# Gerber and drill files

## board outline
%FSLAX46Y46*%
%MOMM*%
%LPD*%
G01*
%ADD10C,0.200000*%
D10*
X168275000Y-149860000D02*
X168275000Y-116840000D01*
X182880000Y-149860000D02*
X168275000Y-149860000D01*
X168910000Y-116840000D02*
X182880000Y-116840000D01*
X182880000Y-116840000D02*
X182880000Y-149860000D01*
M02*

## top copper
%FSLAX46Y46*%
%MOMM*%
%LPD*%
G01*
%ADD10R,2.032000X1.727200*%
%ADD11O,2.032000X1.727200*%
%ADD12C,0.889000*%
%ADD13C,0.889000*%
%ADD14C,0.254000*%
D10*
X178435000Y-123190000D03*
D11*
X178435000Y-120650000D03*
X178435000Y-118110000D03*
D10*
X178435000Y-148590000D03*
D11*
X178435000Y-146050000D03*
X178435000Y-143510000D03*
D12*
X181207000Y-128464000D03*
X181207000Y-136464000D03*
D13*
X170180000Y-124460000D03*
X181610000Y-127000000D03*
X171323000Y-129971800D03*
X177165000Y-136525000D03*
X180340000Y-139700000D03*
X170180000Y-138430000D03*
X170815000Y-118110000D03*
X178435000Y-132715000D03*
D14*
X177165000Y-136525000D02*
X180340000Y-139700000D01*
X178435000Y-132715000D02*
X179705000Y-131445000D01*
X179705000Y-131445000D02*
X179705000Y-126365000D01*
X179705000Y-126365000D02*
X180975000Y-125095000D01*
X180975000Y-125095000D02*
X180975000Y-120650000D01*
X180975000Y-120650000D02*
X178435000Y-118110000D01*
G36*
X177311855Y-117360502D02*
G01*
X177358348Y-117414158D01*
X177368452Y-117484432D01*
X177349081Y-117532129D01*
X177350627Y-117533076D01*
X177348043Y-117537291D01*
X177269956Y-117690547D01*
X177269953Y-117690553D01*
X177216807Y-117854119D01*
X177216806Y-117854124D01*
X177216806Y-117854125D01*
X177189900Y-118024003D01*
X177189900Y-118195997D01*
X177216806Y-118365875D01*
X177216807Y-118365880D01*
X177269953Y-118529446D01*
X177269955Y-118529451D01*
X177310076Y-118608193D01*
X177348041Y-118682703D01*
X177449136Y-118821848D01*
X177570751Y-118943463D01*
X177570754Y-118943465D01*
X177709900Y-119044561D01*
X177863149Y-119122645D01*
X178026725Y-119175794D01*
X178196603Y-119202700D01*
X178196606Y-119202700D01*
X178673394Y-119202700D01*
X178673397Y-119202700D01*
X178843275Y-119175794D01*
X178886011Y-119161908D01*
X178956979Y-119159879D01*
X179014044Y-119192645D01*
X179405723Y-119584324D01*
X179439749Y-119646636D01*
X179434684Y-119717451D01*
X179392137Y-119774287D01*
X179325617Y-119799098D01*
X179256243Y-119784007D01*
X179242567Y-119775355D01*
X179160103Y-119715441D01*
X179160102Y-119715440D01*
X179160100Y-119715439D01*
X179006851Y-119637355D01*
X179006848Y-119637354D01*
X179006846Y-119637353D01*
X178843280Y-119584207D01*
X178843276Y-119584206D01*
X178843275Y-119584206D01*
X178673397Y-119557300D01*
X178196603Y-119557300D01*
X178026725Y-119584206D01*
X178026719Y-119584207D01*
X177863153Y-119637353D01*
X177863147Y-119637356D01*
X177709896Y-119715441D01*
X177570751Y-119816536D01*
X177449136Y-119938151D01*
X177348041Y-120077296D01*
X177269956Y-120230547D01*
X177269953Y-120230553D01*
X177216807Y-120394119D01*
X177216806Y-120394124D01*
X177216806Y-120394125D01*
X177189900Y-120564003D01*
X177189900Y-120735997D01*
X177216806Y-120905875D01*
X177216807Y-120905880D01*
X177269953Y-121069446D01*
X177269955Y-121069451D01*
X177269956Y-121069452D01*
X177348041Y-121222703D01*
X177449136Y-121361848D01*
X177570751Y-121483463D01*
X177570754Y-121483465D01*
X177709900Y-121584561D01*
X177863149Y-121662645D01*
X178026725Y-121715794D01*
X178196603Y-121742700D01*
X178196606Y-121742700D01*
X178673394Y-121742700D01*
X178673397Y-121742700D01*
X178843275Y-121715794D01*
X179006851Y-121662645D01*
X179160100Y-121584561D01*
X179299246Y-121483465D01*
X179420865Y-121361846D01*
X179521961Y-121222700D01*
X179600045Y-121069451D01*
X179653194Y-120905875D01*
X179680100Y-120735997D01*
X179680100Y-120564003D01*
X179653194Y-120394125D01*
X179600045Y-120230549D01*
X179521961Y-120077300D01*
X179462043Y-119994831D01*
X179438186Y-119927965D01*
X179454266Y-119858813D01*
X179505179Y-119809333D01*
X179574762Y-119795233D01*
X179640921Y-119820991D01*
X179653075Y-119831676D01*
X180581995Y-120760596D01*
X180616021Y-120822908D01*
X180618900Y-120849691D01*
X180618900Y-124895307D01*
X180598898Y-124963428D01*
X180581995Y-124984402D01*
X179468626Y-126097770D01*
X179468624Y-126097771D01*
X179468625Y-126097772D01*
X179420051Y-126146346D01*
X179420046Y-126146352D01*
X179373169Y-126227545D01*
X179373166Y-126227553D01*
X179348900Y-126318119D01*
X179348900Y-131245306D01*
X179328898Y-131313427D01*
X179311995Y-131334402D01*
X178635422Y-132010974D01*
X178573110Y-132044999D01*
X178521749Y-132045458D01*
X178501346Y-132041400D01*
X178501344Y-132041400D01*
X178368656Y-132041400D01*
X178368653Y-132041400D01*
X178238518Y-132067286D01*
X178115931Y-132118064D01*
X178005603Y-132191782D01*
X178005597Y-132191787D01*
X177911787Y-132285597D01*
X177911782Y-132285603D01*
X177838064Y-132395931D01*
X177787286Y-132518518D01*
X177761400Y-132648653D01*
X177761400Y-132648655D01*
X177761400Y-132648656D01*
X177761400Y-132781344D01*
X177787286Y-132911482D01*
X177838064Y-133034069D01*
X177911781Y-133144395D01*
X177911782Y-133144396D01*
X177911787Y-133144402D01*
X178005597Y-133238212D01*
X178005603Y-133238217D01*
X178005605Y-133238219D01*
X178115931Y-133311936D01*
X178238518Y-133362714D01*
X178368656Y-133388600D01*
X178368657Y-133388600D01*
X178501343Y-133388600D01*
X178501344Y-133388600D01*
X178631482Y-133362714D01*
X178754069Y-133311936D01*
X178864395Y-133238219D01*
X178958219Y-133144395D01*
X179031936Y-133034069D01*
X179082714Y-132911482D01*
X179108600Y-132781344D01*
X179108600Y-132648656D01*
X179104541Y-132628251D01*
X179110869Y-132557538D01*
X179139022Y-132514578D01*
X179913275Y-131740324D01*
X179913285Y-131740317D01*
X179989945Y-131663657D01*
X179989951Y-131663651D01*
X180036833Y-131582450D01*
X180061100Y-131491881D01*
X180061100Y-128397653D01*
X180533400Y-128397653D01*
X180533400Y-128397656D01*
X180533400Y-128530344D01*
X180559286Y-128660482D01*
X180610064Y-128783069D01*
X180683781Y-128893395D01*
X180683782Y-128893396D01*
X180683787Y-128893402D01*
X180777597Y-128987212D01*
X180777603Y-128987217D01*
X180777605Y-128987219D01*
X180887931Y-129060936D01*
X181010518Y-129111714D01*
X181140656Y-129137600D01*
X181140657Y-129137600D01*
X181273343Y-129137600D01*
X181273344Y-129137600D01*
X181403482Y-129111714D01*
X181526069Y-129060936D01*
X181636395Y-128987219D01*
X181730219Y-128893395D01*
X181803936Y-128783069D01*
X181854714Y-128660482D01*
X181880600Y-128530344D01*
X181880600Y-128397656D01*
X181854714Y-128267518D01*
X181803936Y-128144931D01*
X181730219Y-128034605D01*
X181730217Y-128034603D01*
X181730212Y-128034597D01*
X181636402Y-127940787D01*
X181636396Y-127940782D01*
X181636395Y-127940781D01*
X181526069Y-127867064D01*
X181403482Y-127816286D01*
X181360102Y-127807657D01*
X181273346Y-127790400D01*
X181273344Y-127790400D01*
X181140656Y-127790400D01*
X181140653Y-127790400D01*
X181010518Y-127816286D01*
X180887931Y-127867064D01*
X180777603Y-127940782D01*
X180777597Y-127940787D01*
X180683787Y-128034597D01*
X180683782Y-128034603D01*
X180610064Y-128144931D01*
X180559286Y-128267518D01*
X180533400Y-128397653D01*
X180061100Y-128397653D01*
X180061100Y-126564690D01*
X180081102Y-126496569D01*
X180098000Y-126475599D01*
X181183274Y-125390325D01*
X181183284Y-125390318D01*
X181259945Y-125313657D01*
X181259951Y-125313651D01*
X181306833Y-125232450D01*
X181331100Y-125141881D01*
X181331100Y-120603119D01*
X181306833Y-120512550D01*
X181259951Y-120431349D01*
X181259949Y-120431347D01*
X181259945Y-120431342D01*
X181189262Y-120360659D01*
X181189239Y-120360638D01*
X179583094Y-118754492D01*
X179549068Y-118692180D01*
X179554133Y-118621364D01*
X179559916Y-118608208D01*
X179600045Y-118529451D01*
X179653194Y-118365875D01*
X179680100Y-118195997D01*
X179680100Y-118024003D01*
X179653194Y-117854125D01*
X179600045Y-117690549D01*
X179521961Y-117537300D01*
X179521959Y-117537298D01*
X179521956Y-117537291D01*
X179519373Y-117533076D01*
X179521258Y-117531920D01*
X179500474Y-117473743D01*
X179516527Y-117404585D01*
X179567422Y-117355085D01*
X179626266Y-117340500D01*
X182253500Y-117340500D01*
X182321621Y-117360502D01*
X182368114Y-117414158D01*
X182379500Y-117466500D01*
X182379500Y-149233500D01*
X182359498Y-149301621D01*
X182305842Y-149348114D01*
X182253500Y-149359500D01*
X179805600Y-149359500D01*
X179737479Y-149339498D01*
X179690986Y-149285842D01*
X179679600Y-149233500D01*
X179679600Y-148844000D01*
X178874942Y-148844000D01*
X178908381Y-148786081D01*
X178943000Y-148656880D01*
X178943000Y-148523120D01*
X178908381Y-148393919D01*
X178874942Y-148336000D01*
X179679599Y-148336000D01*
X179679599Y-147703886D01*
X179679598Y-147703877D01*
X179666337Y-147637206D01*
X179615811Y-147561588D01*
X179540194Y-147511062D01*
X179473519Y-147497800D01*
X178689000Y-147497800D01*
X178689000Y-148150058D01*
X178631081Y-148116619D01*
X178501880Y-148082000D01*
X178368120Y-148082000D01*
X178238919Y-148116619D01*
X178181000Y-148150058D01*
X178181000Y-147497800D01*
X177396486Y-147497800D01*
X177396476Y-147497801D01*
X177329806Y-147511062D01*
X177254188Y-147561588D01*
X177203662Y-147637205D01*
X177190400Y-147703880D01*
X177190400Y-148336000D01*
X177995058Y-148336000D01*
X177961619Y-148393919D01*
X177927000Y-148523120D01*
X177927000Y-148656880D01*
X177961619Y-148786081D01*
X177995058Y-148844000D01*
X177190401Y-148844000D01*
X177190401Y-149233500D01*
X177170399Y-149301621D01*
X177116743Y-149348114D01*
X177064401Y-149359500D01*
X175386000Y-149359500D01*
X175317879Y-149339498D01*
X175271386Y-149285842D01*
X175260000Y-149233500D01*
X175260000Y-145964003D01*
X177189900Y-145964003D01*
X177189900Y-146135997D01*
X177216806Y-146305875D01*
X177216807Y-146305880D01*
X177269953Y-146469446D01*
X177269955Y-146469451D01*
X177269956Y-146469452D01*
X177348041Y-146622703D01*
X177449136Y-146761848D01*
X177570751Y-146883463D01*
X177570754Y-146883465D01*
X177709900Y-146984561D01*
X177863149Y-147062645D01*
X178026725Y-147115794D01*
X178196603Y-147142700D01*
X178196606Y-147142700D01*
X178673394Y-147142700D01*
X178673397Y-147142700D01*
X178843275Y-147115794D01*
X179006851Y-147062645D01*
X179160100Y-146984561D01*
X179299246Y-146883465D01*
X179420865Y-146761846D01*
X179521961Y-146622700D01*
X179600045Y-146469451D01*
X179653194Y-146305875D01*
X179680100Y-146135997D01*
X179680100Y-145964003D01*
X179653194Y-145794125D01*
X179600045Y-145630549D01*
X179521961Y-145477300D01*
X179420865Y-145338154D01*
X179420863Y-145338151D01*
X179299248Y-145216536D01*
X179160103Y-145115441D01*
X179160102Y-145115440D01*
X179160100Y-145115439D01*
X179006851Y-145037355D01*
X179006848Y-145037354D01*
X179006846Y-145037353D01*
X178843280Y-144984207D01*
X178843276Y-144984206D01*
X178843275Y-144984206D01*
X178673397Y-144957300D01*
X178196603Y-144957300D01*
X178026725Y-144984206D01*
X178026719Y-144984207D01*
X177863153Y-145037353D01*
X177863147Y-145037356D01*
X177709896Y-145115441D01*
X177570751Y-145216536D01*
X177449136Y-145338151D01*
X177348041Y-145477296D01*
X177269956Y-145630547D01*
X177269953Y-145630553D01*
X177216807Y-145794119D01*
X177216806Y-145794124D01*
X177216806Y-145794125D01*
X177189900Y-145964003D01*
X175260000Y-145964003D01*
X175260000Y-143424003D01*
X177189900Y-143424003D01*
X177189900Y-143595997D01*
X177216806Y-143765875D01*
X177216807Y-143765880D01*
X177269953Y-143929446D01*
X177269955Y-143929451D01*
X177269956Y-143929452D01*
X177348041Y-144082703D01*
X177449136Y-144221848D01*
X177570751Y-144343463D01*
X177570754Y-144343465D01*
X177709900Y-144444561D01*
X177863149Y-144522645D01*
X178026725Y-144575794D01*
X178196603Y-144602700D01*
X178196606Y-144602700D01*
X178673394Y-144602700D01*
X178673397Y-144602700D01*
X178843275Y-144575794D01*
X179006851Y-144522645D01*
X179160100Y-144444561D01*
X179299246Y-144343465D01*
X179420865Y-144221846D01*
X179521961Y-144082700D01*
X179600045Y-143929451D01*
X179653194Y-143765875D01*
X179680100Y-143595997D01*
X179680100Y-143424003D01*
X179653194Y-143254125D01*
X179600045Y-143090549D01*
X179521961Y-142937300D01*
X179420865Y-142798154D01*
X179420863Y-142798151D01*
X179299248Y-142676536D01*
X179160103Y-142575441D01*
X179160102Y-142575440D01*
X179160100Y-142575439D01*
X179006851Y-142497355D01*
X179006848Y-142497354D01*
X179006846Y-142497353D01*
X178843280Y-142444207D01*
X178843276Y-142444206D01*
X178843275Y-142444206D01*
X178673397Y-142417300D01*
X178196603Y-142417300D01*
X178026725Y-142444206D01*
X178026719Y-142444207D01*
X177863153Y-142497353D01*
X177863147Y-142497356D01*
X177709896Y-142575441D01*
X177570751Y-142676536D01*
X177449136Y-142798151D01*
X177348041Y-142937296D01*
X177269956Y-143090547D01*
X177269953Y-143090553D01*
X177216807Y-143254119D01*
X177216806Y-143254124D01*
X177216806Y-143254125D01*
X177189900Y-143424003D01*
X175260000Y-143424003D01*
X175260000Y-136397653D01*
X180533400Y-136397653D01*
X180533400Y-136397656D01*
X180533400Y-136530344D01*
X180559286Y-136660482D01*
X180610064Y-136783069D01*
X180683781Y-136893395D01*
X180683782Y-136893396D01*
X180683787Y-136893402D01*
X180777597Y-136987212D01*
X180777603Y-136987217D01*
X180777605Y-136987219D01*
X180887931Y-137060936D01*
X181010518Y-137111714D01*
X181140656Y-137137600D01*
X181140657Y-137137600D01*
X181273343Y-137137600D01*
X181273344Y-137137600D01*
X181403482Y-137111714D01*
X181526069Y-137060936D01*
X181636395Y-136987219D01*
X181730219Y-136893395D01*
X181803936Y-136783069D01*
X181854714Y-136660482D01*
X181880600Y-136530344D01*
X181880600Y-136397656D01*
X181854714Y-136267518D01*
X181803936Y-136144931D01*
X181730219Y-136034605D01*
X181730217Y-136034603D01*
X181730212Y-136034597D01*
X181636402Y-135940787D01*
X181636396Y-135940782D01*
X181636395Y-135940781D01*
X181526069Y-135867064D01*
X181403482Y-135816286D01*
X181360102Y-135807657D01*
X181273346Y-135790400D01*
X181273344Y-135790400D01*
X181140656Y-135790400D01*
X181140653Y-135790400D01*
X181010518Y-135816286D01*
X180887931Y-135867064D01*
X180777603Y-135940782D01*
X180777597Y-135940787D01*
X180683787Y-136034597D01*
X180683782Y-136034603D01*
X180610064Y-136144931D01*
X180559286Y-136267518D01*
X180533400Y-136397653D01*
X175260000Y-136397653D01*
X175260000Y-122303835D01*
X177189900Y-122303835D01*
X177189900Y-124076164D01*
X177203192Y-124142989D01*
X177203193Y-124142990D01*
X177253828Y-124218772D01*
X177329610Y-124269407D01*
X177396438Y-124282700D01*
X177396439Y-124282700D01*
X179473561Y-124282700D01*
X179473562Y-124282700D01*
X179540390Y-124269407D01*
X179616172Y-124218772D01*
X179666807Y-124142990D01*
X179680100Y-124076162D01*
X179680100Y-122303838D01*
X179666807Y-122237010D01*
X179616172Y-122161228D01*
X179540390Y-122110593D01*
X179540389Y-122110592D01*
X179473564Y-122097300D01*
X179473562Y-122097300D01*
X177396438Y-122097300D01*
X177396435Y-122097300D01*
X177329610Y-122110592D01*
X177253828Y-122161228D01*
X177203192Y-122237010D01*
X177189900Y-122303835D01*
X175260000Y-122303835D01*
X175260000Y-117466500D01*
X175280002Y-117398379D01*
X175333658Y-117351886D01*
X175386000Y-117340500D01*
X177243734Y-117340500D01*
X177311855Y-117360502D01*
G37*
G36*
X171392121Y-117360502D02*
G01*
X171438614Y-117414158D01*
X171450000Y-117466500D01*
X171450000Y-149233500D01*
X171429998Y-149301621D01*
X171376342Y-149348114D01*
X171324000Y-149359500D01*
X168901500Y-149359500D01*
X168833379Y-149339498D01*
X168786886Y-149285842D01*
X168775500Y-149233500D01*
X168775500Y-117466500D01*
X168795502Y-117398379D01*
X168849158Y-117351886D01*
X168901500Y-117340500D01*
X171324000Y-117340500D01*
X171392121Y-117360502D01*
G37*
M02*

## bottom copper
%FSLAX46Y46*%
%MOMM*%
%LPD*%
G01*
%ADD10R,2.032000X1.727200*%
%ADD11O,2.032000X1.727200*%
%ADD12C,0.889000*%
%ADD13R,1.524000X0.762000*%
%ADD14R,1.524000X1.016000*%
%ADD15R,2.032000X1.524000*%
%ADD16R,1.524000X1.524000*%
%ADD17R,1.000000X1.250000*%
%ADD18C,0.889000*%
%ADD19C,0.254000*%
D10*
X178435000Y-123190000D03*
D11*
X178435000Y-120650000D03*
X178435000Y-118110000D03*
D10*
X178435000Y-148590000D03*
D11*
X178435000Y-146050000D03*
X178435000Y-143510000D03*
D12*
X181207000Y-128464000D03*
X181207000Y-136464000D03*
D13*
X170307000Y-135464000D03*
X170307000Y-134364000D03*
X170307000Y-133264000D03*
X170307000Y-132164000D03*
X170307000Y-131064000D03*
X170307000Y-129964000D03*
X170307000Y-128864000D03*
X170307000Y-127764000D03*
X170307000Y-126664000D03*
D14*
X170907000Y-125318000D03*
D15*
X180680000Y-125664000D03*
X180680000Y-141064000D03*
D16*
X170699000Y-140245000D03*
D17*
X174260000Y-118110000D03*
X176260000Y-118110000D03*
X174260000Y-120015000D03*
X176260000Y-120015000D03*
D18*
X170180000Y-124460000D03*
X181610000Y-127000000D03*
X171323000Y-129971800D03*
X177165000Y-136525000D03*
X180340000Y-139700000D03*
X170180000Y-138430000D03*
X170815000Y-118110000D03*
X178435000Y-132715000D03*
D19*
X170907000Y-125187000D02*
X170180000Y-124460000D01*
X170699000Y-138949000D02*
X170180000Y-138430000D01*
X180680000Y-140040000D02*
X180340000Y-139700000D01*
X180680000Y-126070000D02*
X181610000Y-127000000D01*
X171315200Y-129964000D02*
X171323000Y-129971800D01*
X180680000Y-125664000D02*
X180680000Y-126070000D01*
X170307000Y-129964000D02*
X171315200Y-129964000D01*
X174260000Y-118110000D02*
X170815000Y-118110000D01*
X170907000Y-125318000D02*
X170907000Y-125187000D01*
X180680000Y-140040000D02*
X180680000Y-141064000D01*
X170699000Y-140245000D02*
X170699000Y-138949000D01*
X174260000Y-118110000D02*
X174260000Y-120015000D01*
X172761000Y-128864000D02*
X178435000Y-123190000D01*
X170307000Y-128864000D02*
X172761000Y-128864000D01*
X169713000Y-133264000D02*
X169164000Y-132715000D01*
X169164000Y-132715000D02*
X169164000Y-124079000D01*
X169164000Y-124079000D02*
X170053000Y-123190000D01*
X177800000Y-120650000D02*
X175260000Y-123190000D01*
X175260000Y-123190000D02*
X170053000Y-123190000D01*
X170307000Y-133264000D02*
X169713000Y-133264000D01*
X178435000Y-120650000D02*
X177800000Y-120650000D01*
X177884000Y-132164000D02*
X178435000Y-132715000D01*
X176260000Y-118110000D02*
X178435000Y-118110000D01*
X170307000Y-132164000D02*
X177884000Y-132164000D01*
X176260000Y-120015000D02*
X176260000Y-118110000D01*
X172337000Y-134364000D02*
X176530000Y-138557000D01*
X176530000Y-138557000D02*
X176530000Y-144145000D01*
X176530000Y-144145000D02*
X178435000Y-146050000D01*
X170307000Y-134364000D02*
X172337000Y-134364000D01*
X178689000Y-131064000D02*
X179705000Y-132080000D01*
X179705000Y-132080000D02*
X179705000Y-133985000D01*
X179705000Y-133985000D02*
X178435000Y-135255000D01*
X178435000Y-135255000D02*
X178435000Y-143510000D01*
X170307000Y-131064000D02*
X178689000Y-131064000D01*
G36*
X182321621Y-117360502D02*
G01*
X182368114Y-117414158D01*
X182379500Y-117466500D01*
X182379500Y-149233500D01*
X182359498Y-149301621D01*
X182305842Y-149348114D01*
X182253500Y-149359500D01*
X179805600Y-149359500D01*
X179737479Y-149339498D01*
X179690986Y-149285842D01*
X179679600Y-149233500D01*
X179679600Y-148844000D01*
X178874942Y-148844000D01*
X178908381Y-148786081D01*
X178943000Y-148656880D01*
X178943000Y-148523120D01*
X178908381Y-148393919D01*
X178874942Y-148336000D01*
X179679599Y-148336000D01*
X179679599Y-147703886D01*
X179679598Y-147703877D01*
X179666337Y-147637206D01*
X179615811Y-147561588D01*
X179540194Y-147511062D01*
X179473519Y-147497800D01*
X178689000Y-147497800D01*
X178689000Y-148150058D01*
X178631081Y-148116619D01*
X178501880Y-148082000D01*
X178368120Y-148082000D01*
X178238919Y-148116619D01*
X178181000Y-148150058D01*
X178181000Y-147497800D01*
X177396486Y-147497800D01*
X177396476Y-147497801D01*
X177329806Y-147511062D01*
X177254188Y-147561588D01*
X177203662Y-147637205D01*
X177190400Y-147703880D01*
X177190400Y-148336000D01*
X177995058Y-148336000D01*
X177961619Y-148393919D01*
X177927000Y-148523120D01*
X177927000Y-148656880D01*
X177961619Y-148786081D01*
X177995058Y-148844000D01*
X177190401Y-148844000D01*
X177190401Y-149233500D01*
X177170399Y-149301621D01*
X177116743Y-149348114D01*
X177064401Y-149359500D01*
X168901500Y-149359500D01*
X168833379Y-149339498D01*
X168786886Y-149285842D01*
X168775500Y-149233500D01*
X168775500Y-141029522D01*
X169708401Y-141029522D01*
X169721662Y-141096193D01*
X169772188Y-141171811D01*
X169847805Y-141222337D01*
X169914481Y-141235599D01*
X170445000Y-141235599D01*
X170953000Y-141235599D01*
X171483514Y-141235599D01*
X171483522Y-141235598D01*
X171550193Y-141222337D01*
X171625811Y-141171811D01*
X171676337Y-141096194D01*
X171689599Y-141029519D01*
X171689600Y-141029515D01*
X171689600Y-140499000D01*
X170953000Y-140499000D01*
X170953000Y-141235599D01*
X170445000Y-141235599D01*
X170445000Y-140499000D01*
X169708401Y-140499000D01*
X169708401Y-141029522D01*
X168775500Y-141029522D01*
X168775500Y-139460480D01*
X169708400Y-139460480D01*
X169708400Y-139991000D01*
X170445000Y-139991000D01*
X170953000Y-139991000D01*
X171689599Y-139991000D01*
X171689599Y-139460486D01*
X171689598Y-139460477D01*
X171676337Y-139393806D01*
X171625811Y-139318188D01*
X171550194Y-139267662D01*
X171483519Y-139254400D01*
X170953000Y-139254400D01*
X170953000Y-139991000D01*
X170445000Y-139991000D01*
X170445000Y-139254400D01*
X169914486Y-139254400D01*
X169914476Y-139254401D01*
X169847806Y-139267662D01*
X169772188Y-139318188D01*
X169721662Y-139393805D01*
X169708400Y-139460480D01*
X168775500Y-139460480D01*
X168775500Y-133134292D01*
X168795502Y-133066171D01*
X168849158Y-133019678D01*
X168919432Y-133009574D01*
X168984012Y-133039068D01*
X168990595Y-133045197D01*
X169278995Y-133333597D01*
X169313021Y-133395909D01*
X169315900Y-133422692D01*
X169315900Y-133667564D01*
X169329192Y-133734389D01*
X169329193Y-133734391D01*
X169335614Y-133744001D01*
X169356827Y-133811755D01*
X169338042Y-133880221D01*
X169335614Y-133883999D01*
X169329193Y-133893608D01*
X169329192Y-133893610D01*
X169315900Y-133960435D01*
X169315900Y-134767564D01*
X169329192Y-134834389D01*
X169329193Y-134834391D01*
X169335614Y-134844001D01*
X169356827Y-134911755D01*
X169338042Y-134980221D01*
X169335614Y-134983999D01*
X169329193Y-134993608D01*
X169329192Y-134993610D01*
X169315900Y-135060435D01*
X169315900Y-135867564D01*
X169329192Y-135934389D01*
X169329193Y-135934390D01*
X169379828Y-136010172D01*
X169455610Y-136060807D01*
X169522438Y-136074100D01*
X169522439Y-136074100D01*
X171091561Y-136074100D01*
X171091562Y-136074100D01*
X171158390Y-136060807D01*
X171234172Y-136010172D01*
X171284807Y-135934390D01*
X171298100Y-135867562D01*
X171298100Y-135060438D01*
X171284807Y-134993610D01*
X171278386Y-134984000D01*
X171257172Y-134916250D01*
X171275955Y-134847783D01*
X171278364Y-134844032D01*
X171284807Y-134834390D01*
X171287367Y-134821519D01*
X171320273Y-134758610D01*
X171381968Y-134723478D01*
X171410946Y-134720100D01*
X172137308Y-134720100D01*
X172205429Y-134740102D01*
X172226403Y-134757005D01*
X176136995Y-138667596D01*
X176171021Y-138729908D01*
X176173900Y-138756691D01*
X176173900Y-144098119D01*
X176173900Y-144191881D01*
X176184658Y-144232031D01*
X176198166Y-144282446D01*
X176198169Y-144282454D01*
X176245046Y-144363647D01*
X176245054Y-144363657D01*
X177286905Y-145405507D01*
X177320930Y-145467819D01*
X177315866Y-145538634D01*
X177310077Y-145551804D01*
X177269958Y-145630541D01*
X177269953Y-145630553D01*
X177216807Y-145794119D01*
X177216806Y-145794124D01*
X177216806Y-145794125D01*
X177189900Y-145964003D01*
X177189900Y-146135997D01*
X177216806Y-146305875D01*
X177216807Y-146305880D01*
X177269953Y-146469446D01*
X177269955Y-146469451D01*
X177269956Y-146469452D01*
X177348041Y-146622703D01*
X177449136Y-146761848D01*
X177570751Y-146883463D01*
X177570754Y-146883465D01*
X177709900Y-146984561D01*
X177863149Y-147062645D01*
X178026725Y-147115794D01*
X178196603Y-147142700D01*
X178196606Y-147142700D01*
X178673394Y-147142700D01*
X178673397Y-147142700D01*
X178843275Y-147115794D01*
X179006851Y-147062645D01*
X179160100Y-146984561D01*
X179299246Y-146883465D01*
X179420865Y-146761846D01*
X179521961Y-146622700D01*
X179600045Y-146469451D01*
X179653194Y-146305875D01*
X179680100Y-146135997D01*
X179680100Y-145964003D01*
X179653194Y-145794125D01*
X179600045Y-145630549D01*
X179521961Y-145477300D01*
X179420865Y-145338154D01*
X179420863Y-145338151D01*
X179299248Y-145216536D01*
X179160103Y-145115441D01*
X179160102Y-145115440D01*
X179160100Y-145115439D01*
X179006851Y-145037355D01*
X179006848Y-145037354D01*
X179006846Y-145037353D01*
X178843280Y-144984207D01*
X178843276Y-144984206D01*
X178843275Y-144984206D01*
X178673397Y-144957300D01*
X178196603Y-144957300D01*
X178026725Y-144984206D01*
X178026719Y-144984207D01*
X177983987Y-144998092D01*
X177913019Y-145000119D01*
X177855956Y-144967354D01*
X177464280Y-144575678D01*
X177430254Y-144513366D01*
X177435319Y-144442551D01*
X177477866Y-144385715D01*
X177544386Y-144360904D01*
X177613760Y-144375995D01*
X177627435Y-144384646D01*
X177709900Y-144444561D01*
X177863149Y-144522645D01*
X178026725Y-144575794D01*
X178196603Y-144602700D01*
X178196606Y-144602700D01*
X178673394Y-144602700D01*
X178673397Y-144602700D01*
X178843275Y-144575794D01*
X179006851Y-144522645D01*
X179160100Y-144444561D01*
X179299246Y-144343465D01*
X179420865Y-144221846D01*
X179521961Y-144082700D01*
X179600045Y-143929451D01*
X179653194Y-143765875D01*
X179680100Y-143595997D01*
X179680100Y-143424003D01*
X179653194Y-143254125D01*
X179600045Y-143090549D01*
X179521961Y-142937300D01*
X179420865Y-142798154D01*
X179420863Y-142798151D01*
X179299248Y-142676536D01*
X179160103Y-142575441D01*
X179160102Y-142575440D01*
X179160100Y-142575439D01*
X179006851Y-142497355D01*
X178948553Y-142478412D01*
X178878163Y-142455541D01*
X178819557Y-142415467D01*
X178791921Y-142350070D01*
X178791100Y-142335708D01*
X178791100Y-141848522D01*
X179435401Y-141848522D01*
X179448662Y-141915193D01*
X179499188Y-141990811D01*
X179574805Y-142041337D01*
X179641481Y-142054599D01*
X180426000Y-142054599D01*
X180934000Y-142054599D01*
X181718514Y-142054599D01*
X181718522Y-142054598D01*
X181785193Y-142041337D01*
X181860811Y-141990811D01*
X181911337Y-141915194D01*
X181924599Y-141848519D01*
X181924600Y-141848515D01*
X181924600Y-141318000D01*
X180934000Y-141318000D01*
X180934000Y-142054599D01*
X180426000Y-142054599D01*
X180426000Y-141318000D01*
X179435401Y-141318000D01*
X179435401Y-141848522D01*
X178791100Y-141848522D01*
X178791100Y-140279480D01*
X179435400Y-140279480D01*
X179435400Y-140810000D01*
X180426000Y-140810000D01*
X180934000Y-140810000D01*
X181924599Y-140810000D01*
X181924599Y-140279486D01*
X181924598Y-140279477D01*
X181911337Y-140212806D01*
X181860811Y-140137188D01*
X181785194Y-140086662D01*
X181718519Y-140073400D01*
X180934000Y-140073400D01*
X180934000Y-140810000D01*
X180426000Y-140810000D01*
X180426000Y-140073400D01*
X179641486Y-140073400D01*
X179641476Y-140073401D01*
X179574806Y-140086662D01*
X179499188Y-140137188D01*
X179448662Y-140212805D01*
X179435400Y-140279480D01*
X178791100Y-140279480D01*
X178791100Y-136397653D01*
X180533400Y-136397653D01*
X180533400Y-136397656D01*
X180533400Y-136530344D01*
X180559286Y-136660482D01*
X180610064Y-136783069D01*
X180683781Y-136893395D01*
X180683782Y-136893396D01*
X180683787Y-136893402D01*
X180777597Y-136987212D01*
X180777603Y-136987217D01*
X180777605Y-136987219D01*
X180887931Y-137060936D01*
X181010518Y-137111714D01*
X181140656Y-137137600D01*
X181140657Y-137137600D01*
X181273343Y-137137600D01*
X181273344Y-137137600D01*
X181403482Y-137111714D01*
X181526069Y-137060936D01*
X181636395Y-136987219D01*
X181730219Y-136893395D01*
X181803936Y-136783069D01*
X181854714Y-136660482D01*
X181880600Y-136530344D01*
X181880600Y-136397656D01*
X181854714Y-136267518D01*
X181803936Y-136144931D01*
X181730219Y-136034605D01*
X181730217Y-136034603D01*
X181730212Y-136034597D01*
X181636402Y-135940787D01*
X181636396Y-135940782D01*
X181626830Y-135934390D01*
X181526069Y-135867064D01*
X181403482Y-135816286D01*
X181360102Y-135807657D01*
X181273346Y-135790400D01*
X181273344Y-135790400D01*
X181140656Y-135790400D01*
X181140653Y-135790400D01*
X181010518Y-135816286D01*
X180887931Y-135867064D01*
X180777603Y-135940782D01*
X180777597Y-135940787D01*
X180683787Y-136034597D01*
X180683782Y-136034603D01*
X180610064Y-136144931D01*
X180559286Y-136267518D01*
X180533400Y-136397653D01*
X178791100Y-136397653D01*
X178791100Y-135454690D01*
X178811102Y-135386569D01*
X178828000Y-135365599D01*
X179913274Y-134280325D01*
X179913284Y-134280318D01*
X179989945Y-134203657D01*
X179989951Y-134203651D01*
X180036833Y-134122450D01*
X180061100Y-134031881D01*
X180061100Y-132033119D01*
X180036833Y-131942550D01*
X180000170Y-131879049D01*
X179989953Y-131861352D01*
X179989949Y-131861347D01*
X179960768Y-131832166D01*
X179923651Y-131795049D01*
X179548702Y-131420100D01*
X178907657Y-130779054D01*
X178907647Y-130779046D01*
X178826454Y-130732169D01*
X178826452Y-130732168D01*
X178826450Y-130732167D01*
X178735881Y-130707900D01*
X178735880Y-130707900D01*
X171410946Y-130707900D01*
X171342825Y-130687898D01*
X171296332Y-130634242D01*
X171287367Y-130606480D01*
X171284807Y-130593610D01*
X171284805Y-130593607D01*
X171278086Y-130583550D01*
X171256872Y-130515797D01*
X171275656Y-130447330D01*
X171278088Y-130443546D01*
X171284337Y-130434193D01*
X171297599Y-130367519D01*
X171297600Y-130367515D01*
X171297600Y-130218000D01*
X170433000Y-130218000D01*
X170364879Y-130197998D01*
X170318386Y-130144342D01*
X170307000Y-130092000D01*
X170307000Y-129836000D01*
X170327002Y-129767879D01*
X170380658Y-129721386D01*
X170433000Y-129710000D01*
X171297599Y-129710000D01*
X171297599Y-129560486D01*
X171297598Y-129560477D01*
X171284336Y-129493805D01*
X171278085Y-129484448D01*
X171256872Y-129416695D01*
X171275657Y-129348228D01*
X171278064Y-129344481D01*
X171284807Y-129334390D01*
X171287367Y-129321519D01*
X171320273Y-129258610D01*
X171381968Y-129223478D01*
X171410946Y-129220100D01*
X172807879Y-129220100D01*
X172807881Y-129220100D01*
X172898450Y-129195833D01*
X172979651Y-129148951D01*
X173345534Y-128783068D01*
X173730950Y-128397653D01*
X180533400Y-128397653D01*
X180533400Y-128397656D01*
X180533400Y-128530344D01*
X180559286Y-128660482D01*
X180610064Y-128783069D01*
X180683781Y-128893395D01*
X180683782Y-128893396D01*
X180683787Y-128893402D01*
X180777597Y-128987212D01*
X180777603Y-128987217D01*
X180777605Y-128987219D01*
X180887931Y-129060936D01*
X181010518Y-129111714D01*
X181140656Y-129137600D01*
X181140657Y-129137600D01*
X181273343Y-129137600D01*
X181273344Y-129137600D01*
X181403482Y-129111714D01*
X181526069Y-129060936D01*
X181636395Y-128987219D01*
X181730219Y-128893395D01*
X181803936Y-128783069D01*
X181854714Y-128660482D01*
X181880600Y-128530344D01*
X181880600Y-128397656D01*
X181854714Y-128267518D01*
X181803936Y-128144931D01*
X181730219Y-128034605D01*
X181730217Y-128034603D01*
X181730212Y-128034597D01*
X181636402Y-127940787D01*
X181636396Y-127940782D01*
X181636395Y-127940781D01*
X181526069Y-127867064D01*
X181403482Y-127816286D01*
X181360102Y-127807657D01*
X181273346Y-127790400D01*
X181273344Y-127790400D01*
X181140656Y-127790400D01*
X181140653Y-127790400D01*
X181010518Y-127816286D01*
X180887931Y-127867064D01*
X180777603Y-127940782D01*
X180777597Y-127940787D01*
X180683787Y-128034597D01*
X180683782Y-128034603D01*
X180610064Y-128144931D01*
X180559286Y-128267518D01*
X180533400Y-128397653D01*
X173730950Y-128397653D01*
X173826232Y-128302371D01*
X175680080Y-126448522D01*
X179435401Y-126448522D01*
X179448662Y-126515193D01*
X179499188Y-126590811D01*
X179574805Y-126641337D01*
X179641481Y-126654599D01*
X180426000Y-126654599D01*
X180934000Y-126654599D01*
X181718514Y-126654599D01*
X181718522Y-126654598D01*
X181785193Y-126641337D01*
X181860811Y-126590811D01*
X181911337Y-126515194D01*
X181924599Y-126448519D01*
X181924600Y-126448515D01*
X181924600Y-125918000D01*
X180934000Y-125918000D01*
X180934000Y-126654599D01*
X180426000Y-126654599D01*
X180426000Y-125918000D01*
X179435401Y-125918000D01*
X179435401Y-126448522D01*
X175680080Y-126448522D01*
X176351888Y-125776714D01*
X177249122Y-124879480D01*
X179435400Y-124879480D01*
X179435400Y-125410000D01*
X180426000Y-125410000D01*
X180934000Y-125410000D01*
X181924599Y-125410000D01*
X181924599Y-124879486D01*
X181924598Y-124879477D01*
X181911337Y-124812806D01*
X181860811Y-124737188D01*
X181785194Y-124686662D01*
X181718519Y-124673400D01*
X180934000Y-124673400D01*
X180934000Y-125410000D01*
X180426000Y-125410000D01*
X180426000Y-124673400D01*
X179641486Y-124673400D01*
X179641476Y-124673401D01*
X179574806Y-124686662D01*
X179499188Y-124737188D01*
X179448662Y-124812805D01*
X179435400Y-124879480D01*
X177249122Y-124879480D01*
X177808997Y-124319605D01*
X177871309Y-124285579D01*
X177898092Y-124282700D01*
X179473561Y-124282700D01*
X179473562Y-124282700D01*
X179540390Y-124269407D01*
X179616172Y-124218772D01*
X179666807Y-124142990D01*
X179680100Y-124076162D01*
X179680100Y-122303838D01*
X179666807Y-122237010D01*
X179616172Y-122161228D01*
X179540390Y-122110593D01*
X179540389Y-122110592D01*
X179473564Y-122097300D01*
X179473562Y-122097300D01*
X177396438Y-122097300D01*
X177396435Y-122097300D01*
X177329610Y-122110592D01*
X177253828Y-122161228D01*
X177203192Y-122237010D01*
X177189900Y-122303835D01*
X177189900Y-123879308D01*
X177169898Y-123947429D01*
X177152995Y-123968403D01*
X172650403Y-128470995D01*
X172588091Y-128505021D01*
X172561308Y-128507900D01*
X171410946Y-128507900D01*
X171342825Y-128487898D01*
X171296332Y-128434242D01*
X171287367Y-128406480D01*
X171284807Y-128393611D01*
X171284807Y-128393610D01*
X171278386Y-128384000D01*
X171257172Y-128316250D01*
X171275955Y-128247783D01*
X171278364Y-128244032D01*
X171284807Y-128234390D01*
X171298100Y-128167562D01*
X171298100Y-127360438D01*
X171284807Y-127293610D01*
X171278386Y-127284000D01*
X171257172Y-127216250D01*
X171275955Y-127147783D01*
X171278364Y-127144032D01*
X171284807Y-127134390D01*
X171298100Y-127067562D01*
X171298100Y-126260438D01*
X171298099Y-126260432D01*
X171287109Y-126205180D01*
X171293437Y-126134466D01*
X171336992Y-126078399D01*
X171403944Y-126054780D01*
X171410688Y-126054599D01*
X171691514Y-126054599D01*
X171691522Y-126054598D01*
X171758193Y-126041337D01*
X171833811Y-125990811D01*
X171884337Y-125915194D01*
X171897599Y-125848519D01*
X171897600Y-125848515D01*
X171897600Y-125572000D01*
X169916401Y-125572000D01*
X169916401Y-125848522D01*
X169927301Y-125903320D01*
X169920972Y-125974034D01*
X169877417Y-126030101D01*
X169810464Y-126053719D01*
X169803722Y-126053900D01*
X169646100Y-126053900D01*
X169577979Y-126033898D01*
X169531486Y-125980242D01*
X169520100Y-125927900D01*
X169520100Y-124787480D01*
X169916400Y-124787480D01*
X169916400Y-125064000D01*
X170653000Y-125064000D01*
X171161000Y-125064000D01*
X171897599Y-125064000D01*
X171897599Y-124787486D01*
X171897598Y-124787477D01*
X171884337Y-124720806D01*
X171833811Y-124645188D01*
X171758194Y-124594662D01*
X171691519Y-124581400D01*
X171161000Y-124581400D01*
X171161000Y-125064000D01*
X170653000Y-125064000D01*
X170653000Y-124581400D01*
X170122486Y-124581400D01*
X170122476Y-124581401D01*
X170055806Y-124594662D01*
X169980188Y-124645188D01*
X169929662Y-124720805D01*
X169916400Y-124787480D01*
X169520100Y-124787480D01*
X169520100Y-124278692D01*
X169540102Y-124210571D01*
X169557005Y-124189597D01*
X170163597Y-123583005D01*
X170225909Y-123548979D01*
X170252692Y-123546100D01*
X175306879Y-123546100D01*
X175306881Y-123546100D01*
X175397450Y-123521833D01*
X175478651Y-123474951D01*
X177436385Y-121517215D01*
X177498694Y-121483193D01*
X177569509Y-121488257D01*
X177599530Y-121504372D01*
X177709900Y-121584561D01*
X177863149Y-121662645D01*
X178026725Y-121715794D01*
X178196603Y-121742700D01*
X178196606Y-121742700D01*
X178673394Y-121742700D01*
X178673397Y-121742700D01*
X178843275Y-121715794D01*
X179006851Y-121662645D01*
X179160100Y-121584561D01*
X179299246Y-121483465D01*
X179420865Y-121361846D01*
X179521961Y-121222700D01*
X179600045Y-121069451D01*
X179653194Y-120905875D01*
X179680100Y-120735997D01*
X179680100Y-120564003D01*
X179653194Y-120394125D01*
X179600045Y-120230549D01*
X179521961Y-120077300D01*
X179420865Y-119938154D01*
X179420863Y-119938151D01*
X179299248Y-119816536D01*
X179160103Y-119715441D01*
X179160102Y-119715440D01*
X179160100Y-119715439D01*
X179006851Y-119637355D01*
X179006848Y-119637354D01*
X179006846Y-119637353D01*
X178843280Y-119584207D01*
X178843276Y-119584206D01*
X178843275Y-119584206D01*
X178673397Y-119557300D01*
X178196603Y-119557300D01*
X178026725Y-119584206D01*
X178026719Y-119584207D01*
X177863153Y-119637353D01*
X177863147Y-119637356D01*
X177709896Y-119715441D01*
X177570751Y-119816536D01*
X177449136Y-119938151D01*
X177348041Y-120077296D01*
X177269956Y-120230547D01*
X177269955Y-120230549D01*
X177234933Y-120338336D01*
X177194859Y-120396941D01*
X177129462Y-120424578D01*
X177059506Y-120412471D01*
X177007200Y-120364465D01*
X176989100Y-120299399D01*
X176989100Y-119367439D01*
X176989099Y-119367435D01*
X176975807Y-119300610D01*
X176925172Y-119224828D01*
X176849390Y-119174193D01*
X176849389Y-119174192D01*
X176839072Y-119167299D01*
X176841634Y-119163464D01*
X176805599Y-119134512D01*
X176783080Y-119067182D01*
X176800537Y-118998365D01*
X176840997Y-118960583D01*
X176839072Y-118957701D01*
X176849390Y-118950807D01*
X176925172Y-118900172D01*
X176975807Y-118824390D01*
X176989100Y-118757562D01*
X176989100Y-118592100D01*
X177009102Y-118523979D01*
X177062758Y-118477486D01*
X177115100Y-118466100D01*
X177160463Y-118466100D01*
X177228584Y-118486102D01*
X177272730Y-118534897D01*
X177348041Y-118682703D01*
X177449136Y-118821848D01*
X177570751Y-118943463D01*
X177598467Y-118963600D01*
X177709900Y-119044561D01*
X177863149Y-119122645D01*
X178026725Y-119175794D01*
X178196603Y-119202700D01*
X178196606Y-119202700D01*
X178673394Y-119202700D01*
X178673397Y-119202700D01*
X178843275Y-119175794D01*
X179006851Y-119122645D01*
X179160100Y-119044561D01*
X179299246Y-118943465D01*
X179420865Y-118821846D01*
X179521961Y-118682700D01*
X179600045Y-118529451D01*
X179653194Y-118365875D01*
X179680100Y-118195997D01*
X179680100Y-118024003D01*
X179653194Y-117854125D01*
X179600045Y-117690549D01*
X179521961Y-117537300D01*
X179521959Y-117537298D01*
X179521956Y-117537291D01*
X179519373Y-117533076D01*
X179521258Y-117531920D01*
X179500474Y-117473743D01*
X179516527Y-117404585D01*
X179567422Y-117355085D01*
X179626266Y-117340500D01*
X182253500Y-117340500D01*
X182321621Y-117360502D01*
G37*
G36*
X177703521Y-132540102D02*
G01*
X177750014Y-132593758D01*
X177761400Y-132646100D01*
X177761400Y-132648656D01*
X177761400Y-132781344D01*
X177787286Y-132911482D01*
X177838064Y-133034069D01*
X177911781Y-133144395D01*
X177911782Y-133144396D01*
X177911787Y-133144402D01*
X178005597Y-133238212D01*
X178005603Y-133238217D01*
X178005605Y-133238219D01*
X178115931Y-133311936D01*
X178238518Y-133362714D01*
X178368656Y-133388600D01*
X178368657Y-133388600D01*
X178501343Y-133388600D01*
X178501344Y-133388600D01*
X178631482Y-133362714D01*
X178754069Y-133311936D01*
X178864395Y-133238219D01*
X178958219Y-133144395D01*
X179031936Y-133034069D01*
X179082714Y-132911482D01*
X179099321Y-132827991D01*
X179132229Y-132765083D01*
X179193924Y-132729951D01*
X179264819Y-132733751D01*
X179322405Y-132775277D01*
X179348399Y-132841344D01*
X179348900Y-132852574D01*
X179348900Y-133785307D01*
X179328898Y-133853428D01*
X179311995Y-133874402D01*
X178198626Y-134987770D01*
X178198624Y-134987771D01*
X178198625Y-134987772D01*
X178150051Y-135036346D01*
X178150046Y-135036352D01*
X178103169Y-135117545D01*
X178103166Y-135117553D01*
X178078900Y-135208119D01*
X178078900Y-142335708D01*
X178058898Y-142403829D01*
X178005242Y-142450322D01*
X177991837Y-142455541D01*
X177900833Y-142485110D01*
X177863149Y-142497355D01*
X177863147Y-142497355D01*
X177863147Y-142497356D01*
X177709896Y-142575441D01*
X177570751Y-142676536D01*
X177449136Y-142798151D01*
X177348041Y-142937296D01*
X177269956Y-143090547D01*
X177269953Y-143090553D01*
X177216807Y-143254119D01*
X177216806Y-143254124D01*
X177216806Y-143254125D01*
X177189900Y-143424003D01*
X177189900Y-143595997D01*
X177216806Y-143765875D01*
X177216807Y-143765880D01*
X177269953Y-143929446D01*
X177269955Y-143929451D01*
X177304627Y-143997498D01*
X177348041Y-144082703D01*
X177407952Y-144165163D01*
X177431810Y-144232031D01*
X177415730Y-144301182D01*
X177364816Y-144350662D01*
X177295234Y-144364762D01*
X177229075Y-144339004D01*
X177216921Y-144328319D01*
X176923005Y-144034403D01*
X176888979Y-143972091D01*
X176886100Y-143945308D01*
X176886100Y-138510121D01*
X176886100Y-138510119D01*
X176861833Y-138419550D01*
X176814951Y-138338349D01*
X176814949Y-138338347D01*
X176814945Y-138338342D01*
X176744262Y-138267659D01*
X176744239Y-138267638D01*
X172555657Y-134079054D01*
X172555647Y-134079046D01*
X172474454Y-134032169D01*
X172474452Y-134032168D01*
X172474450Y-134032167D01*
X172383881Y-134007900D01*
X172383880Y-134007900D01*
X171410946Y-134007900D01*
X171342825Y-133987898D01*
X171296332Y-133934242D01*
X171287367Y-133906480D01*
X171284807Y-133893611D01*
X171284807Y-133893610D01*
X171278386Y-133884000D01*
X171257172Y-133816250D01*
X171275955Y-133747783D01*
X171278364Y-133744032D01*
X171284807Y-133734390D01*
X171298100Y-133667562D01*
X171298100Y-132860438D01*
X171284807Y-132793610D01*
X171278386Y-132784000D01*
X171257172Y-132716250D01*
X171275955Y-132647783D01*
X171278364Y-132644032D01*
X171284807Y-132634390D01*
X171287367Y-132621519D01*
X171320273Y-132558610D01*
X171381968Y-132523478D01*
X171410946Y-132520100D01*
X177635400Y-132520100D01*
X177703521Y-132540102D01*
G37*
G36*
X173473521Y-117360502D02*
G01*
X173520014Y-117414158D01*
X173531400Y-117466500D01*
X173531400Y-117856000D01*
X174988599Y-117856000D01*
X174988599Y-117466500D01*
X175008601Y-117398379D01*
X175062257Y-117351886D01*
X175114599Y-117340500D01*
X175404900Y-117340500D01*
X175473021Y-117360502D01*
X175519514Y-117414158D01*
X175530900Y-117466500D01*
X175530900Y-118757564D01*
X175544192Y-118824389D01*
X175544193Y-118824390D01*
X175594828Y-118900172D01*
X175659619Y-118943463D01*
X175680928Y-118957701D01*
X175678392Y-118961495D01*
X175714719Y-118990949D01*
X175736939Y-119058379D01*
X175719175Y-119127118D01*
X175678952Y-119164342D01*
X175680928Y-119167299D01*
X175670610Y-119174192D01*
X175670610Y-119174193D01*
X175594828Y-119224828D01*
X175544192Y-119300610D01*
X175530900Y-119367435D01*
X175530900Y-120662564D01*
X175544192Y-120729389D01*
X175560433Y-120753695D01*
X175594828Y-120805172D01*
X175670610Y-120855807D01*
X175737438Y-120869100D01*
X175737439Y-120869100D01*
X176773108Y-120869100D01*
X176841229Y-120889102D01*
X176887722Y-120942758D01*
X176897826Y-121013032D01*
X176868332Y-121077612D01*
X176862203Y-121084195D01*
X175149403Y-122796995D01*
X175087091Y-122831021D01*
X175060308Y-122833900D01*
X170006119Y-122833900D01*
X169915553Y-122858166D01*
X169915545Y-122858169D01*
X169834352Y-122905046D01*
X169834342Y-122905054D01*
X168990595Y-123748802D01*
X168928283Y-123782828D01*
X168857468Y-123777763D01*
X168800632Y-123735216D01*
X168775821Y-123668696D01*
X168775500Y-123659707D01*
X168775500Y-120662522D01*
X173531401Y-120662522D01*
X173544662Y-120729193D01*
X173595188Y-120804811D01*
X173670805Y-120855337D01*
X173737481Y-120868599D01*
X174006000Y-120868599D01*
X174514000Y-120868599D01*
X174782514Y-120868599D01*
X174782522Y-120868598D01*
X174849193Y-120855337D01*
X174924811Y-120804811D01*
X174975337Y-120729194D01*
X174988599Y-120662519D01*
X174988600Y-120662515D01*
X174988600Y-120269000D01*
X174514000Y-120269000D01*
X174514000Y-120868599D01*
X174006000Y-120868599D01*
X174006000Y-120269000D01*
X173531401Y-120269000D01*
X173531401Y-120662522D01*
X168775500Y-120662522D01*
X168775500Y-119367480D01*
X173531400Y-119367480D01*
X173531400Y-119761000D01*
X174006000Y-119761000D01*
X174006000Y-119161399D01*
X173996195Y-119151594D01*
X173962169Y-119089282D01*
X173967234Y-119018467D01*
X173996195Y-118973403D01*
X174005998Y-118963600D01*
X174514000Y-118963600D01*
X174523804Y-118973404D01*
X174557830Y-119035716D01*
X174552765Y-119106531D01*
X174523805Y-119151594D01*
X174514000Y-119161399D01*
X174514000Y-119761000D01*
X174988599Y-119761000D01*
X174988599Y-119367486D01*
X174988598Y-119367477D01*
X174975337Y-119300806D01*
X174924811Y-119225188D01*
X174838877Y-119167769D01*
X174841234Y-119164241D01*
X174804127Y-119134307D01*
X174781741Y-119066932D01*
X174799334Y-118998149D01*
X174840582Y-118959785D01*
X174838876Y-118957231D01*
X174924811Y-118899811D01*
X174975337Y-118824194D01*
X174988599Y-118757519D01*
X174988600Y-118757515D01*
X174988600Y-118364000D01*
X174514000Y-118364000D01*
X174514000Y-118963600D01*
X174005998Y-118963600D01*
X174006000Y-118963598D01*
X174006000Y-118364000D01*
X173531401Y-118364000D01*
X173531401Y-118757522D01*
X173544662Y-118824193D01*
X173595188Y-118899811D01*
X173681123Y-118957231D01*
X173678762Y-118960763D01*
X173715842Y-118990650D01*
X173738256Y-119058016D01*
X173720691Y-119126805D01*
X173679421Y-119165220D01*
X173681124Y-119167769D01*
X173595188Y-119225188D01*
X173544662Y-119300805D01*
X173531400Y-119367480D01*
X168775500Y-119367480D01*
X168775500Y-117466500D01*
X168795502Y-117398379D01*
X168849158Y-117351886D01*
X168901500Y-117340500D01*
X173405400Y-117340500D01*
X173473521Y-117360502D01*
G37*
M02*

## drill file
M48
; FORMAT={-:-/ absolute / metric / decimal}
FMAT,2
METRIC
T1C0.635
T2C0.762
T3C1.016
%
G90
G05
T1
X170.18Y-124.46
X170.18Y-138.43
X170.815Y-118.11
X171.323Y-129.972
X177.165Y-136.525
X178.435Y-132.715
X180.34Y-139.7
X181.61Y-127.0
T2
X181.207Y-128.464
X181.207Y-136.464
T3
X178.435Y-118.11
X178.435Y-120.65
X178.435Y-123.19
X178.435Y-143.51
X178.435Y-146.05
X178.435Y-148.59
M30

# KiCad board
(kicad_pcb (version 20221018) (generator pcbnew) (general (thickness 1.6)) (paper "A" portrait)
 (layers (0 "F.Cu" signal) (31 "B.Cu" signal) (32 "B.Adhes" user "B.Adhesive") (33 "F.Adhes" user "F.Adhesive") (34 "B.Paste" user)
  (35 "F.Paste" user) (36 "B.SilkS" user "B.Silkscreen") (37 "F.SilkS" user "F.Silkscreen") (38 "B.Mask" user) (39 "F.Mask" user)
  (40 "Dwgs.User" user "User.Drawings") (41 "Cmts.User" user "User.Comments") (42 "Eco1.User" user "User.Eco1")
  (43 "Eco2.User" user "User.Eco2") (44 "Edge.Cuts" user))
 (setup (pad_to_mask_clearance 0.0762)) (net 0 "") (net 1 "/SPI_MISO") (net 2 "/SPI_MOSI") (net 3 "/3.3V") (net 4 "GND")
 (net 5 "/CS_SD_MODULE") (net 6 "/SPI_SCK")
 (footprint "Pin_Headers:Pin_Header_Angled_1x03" (layer "F.Cu") (at 178.435 123.19 180)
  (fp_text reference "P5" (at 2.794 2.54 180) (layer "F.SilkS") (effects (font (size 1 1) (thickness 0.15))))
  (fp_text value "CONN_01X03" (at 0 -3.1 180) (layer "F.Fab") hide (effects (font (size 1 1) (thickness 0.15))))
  (pad "1" thru_hole rect (at 0 0 180) (size 2.032 1.7272) (drill 1.016) (layers "*.Cu" "*.Mask") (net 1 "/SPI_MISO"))
  (pad "2" thru_hole oval (at 0 2.54 180) (size 2.032 1.7272) (drill 1.016) (layers "*.Cu" "*.Mask") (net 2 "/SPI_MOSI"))
  (pad "3" thru_hole oval (at 0 5.08 180) (size 2.032 1.7272) (drill 1.016) (layers "*.Cu" "*.Mask") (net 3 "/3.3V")))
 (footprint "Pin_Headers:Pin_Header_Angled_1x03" (layer "F.Cu") (at 178.435 148.59 180)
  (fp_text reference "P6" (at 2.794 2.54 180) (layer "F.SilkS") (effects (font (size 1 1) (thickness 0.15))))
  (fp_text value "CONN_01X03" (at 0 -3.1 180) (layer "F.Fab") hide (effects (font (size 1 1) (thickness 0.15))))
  (pad "1" thru_hole rect (at 0 0 180) (size 2.032 1.7272) (drill 1.016) (layers "*.Cu" "*.Mask") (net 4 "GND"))
  (pad "2" thru_hole oval (at 0 2.54 180) (size 2.032 1.7272) (drill 1.016) (layers "*.Cu" "*.Mask") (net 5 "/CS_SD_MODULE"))
  (pad "3" thru_hole oval (at 0 5.08 180) (size 2.032 1.7272) (drill 1.016) (layers "*.Cu" "*.Mask") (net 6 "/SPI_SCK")))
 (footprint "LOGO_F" (layer "F.Cu") (at 175.895 137.16)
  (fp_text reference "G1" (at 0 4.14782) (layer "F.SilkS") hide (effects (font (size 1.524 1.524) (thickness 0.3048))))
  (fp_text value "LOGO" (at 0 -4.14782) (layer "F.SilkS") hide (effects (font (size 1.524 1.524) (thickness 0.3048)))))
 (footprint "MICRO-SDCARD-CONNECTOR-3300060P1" (layer "B.Cu") (at 177.8 133.35)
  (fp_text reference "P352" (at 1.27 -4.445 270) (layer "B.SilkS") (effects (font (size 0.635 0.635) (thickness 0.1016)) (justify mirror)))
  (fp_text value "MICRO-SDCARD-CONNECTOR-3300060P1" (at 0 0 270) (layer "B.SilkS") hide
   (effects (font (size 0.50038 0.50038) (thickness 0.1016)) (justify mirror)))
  (pad "" thru_hole circle (at 3.407 -4.886) (size 0.889 0.889) (drill 0.762) (layers "*.Cu" "*.Mask" "B.SilkS"))
  (pad "" thru_hole circle (at 3.407 3.114) (size 0.889 0.889) (drill 0.762) (layers "*.Cu" "*.Mask" "B.SilkS"))
  (pad "1" smd rect (at -7.493 2.114) (size 1.524 0.762) (layers "B.Cu" "B.Paste" "B.Mask"))
  (pad "2" smd rect (at -7.493 1.014) (size 1.524 0.762) (layers "B.Cu" "B.Paste" "B.Mask") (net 5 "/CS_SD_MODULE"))
  (pad "3" smd rect (at -7.493 -0.086) (size 1.524 0.762) (layers "B.Cu" "B.Paste" "B.Mask") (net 2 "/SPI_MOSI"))
  (pad "4" smd rect (at -7.493 -1.186) (size 1.524 0.762) (layers "B.Cu" "B.Paste" "B.Mask") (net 3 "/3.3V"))
  (pad "5" smd rect (at -7.493 -2.286) (size 1.524 0.762) (layers "B.Cu" "B.Paste" "B.Mask") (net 6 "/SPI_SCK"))
  (pad "6" smd rect (at -7.493 -3.386) (size 1.524 0.762) (layers "B.Cu" "B.Paste" "B.Mask") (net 4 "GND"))
  (pad "7" smd rect (at -7.493 -4.486) (size 1.524 0.762) (layers "B.Cu" "B.Paste" "B.Mask") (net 1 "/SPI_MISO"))
  (pad "8" smd rect (at -7.493 -5.586) (size 1.524 0.762) (layers "B.Cu" "B.Paste" "B.Mask"))
  (pad "9" smd rect (at -7.493 -6.686) (size 1.524 0.762) (layers "B.Cu" "B.Paste" "B.Mask"))
  (pad "G1" smd rect (at -6.893 -8.032) (size 1.524 1.016) (layers "B.Cu" "B.Paste" "B.Mask") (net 4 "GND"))
  (pad "G2" smd rect (at 2.88 -7.686) (size 2.032 1.524) (layers "B.Cu" "B.Paste" "B.Mask") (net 4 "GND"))
  (pad "G3" smd rect (at 2.88 7.714) (size 2.032 1.524) (layers "B.Cu" "B.Paste" "B.Mask") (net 4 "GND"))
  (pad "G4" smd rect (at -7.101 6.895) (size 1.524 1.524) (layers "B.Cu" "B.Paste" "B.Mask") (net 4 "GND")))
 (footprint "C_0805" (layer "B.Cu") (at 175.26 118.11)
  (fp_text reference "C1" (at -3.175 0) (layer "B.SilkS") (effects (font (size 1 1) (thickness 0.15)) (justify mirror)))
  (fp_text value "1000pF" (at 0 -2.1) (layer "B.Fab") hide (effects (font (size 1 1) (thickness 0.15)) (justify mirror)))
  (pad "1" smd rect (at -1 0) (size 1 1.25) (layers "B.Cu" "B.Paste" "B.Mask") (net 4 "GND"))
  (pad "2" smd rect (at 1 0) (size 1 1.25) (layers "B.Cu" "B.Paste" "B.Mask") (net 3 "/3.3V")))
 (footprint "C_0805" (layer "B.Cu") (at 175.26 120.015)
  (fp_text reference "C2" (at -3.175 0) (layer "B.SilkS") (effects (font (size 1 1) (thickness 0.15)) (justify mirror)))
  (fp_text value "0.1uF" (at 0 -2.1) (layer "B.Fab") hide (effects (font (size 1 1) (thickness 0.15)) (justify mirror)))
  (pad "1" smd rect (at -1 0) (size 1 1.25) (layers "B.Cu" "B.Paste" "B.Mask") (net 4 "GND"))
  (pad "2" smd rect (at 1 0) (size 1 1.25) (layers "B.Cu" "B.Paste" "B.Mask") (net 3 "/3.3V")))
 (gr_line (start 168.275 149.86) (end 168.275 116.84) (stroke (width 0.2) (type solid)) (layer "Edge.Cuts"))
 (gr_line (start 182.88 149.86) (end 168.275 149.86) (stroke (width 0.2) (type solid)) (layer "Edge.Cuts"))
 (gr_line (start 168.91 116.84) (end 182.88 116.84) (stroke (width 0.2) (type solid)) (layer "Edge.Cuts"))
 (gr_line (start 182.88 116.84) (end 182.88 149.86) (stroke (width 0.2) (type solid)) (layer "Edge.Cuts"))
 (segment (start 177.165 136.525) (end 180.34 139.7) (width 0.254) (layer "F.Cu") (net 4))
 (via (at 170.18 124.46) (size 0.889) (drill 0.635) (layers "F.Cu" "B.Cu") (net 4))
 (via (at 181.61 127) (size 0.889) (drill 0.635) (layers "F.Cu" "B.Cu") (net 4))
 (via (at 171.323 129.9718) (size 0.889) (drill 0.635) (layers "F.Cu" "B.Cu") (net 4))
 (via (at 177.165 136.525) (size 0.889) (drill 0.635) (layers "F.Cu" "B.Cu") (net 4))
 (via (at 180.34 139.7) (size 0.889) (drill 0.635) (layers "F.Cu" "B.Cu") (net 4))
 (via (at 170.18 138.43) (size 0.889) (drill 0.635) (layers "F.Cu" "B.Cu") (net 4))
 (via (at 170.815 118.11) (size 0.889) (drill 0.635) (layers "F.Cu" "B.Cu") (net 4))
 (segment (start 170.907 125.187) (end 170.18 124.46) (width 0.254) (layer "B.Cu") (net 4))
 (segment (start 170.699 138.949) (end 170.18 138.43) (width 0.254) (layer "B.Cu") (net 4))
 (segment (start 180.68 140.04) (end 180.34 139.7) (width 0.254) (layer "B.Cu") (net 4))
 (segment (start 180.68 126.07) (end 181.61 127) (width 0.254) (layer "B.Cu") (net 4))
 (segment (start 171.3152 129.964) (end 171.323 129.9718) (width 0.254) (layer "B.Cu") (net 4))
 (segment (start 180.68 125.664) (end 180.68 126.07) (width 0.254) (layer "B.Cu") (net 4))
 (segment (start 170.307 129.964) (end 171.3152 129.964) (width 0.254) (layer "B.Cu") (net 4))
 (segment (start 174.26 118.11) (end 170.815 118.11) (width 0.254) (layer "B.Cu") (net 4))
 (segment (start 170.907 125.318) (end 170.907 125.187) (width 0.254) (layer "B.Cu") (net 4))
 (segment (start 180.68 140.04) (end 180.68 141.064) (width 0.254) (layer "B.Cu") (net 4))
 (segment (start 170.699 140.245) (end 170.699 138.949) (width 0.254) (layer "B.Cu") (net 4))
 (segment (start 174.26 118.11) (end 174.26 120.015) (width 0.254) (layer "B.Cu") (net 4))
 (segment (start 172.761 128.864) (end 178.435 123.19) (width 0.254) (layer "B.Cu") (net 1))
 (segment (start 170.307 128.864) (end 172.761 128.864) (width 0.254) (layer "B.Cu") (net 1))
 (segment (start 169.713 133.264) (end 169.164 132.715) (width 0.254) (layer "B.Cu") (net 2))
 (segment (start 169.164 132.715) (end 169.164 124.079) (width 0.254) (layer "B.Cu") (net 2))
 (segment (start 169.164 124.079) (end 170.053 123.19) (width 0.254) (layer "B.Cu") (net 2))
 (segment (start 177.8 120.65) (end 175.26 123.19) (width 0.254) (layer "B.Cu") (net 2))
 (segment (start 175.26 123.19) (end 170.053 123.19) (width 0.254) (layer "B.Cu") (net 2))
 (segment (start 170.307 133.264) (end 169.713 133.264) (width 0.254) (layer "B.Cu") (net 2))
 (segment (start 178.435 120.65) (end 177.8 120.65) (width 0.254) (layer "B.Cu") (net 2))
 (segment (start 178.435 132.715) (end 179.705 131.445) (width 0.254) (layer "F.Cu") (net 3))
 (segment (start 179.705 131.445) (end 179.705 126.365) (width 0.254) (layer "F.Cu") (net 3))
 (segment (start 179.705 126.365) (end 180.975 125.095) (width 0.254) (layer "F.Cu") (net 3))
 (segment (start 180.975 125.095) (end 180.975 120.65) (width 0.254) (layer "F.Cu") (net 3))
 (segment (start 180.975 120.65) (end 178.435 118.11) (width 0.254) (layer "F.Cu") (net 3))
 (via (at 178.435 132.715) (size 0.889) (drill 0.635) (layers "F.Cu" "B.Cu") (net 3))
 (segment (start 177.884 132.164) (end 178.435 132.715) (width 0.254) (layer "B.Cu") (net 3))
 (segment (start 176.26 118.11) (end 178.435 118.11) (width 0.254) (layer "B.Cu") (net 3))
 (segment (start 170.307 132.164) (end 177.884 132.164) (width 0.254) (layer "B.Cu") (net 3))
 (segment (start 176.26 120.015) (end 176.26 118.11) (width 0.254) (layer "B.Cu") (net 3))
 (segment (start 172.337 134.364) (end 176.53 138.557) (width 0.254) (layer "B.Cu") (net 5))
 (segment (start 176.53 138.557) (end 176.53 144.145) (width 0.254) (layer "B.Cu") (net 5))
 (segment (start 176.53 144.145) (end 178.435 146.05) (width 0.254) (layer "B.Cu") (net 5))
 (segment (start 170.307 134.364) (end 172.337 134.364) (width 0.254) (layer "B.Cu") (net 5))
 (segment (start 178.689 131.064) (end 179.705 132.08) (width 0.254) (layer "B.Cu") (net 6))
 (segment (start 179.705 132.08) (end 179.705 133.985) (width 0.254) (layer "B.Cu") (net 6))
 (segment (start 179.705 133.985) (end 178.435 135.255) (width 0.254) (layer "B.Cu") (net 6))
 (segment (start 178.435 135.255) (end 178.435 143.51) (width 0.254) (layer "B.Cu") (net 6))
 (segment (start 170.307 131.064) (end 178.689 131.064) (width 0.254) (layer "B.Cu") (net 6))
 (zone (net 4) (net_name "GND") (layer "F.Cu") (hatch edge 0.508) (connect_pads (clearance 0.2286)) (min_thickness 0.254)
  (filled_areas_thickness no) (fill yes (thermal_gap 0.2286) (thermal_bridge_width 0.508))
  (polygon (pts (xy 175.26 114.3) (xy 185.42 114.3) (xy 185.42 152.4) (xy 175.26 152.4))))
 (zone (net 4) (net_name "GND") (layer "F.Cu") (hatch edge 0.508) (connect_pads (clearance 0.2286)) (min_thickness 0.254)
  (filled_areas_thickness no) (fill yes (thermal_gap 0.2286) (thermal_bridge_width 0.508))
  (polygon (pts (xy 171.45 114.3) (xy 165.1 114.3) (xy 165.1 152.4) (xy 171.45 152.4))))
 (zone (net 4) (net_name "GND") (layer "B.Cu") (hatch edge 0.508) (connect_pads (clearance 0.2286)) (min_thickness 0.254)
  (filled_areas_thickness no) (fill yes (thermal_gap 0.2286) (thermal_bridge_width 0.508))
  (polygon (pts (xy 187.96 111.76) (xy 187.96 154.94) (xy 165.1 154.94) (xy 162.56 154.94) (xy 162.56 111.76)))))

